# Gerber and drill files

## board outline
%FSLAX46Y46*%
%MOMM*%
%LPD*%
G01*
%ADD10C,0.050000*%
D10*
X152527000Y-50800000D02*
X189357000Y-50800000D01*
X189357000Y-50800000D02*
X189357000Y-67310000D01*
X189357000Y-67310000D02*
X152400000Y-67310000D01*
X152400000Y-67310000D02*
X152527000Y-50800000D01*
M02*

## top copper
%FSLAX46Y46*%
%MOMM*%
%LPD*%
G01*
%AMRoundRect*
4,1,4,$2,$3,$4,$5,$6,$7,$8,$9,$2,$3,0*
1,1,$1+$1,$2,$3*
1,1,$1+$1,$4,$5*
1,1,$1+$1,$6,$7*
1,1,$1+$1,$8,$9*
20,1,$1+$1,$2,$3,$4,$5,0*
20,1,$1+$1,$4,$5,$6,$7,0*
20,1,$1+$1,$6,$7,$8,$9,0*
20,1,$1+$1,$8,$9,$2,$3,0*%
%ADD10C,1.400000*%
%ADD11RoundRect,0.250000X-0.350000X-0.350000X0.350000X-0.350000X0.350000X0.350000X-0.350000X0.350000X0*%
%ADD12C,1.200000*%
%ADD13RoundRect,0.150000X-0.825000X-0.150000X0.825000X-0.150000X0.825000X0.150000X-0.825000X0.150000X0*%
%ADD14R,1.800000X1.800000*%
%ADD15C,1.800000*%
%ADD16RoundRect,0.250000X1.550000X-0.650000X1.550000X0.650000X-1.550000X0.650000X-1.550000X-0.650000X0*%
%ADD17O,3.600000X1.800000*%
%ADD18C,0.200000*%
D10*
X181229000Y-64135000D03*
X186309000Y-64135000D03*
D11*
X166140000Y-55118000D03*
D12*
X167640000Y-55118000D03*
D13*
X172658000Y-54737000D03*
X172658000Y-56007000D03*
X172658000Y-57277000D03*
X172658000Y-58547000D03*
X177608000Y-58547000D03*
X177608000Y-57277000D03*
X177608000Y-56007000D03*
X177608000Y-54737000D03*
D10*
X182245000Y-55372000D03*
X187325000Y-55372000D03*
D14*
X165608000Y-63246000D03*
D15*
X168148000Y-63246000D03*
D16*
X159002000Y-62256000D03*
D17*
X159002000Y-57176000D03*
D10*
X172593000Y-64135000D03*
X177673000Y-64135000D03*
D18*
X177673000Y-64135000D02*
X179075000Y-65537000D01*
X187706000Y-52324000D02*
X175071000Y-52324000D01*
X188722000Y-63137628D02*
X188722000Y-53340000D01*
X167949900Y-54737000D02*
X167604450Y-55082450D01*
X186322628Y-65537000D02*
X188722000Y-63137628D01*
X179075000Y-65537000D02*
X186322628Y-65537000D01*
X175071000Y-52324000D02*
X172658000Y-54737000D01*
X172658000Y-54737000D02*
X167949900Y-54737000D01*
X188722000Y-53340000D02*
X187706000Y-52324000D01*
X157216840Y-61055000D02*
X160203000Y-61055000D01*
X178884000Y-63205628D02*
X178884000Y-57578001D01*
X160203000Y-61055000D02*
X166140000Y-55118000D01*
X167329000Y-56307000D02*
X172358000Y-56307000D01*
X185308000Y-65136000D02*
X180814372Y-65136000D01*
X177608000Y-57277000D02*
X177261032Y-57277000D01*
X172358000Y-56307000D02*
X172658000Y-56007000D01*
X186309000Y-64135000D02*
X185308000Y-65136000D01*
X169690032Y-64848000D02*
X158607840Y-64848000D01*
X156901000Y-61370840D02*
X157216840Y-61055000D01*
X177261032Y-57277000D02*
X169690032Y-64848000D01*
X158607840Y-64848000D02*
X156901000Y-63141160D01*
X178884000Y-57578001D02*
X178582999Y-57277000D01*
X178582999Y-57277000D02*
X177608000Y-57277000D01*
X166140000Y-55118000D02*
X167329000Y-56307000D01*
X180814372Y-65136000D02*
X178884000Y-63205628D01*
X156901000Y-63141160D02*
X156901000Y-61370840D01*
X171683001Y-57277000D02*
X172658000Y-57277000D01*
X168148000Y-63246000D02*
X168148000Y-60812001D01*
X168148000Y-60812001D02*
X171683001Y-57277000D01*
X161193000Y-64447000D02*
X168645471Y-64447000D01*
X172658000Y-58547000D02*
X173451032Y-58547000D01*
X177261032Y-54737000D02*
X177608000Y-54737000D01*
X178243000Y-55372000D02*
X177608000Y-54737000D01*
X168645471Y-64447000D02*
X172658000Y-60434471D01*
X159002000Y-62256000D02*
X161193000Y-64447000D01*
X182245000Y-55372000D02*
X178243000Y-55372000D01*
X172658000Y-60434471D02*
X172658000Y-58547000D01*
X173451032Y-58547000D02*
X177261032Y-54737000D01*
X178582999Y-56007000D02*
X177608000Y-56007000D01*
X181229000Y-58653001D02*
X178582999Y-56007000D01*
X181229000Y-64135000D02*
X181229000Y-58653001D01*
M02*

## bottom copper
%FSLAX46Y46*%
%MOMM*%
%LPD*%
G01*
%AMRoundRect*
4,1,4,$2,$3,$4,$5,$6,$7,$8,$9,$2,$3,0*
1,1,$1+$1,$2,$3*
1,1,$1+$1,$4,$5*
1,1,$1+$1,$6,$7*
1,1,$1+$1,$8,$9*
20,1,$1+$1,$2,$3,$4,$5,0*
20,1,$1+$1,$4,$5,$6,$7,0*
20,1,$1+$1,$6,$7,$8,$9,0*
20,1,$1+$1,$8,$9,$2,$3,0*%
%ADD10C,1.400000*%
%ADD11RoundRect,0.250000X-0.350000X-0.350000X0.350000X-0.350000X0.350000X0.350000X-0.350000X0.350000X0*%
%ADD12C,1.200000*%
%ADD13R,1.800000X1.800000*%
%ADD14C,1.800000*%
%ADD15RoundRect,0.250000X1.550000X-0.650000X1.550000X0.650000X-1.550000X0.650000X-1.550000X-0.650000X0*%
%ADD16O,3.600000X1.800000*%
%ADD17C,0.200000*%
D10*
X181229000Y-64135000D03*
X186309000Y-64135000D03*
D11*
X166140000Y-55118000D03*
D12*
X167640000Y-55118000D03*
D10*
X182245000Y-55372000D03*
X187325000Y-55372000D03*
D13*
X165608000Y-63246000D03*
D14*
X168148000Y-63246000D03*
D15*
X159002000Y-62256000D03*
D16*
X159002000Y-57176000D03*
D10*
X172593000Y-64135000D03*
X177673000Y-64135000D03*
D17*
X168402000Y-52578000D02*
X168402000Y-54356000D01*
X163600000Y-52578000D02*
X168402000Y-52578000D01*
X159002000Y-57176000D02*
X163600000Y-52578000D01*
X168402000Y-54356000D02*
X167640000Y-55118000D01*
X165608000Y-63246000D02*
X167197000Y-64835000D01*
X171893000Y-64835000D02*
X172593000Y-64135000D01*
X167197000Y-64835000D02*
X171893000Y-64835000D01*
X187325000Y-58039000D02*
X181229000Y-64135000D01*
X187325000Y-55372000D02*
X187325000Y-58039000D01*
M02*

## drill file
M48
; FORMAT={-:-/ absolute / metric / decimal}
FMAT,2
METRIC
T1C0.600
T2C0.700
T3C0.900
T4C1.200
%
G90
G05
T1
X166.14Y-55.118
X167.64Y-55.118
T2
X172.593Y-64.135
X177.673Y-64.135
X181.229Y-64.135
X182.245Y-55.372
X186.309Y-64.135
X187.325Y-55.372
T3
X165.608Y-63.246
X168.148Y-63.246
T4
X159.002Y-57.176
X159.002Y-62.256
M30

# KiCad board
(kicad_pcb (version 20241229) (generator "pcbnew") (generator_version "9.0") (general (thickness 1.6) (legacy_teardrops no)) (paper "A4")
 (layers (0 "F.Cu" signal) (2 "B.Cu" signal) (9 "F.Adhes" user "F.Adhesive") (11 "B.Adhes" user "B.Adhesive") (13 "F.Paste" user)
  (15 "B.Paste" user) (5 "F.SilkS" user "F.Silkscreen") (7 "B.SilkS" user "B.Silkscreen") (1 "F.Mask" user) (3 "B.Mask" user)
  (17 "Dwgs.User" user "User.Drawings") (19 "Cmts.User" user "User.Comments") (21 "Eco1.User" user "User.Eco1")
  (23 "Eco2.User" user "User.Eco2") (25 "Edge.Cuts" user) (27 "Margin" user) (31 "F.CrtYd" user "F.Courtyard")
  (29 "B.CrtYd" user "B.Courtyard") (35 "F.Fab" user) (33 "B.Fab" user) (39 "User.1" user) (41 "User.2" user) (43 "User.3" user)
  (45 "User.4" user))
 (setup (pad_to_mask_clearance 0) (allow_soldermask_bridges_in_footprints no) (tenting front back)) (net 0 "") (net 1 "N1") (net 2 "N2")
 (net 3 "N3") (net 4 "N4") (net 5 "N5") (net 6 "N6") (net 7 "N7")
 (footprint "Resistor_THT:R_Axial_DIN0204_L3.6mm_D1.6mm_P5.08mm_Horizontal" (layer "F.Cu") (at 181.229 64.135)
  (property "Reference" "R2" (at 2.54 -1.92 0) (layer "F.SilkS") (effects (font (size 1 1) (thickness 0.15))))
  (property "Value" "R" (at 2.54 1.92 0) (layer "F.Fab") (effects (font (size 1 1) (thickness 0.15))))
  (pad "1" thru_hole circle (at 0 0) (size 1.4 1.4) (drill 0.7) (layers "*.Cu" "*.Mask") (remove_unused_layers no) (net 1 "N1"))
  (pad "2" thru_hole circle (at 5.08 0) (size 1.4 1.4) (drill 0.7) (layers "*.Cu" "*.Mask") (remove_unused_layers no) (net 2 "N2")))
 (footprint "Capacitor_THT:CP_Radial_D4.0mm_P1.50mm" (layer "F.Cu") (at 166.14 55.118)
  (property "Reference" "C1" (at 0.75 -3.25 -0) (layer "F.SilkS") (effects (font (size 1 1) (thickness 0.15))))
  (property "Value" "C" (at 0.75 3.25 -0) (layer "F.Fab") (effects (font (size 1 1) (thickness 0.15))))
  (pad "1" thru_hole roundrect (at 0 0) (size 1.2 1.2) (drill 0.6) (layers "*.Cu" "*.Mask") (remove_unused_layers no)
   (roundrect_rratio 0.208333) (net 2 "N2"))
  (pad "2" thru_hole circle (at 1.5 0) (size 1.2 1.2) (drill 0.6) (layers "*.Cu" "*.Mask") (remove_unused_layers no) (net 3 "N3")))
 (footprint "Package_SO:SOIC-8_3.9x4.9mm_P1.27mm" (layer "F.Cu") (at 175.133 56.642)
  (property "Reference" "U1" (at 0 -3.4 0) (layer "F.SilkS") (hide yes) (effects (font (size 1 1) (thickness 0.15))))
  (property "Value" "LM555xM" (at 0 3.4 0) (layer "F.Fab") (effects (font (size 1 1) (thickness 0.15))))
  (pad "1" smd roundrect (at -2.475 -1.905) (size 1.95 0.6) (layers "F.Cu" "F.Mask" "F.Paste") (roundrect_rratio 0.25) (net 3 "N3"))
  (pad "2" smd roundrect (at -2.475 -0.635) (size 1.95 0.6) (layers "F.Cu" "F.Mask" "F.Paste") (roundrect_rratio 0.25) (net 2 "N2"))
  (pad "3" smd roundrect (at -2.475 0.635) (size 1.95 0.6) (layers "F.Cu" "F.Mask" "F.Paste") (roundrect_rratio 0.25) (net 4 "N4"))
  (pad "4" smd roundrect (at -2.475 1.905) (size 1.95 0.6) (layers "F.Cu" "F.Mask" "F.Paste") (roundrect_rratio 0.25) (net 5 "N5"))
  (pad "5" smd roundrect (at 2.475 1.905) (size 1.95 0.6) (layers "F.Cu" "F.Mask" "F.Paste") (roundrect_rratio 0.25) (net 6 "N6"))
  (pad "6" smd roundrect (at 2.475 0.635) (size 1.95 0.6) (layers "F.Cu" "F.Mask" "F.Paste") (roundrect_rratio 0.25) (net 2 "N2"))
  (pad "7" smd roundrect (at 2.475 -0.635) (size 1.95 0.6) (layers "F.Cu" "F.Mask" "F.Paste") (roundrect_rratio 0.25) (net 1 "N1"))
  (pad "8" smd roundrect (at 2.475 -1.905) (size 1.95 0.6) (layers "F.Cu" "F.Mask" "F.Paste") (roundrect_rratio 0.25) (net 5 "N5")))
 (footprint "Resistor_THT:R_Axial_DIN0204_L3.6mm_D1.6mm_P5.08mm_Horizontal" (layer "F.Cu") (at 182.245 55.372)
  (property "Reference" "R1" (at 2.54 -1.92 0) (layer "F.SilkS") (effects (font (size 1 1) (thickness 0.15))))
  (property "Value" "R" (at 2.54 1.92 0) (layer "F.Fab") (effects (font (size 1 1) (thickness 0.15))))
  (pad "1" thru_hole circle (at 0 0) (size 1.4 1.4) (drill 0.7) (layers "*.Cu" "*.Mask") (remove_unused_layers no) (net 5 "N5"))
  (pad "2" thru_hole circle (at 5.08 0) (size 1.4 1.4) (drill 0.7) (layers "*.Cu" "*.Mask") (remove_unused_layers no) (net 1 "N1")))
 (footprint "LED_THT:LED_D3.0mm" (layer "F.Cu") (at 165.608 63.246)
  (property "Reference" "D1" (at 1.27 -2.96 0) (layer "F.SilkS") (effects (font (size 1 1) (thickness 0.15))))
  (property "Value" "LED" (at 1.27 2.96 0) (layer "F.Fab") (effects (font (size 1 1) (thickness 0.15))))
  (pad "1" thru_hole rect (at 0 0) (size 1.8 1.8) (drill 0.9) (layers "*.Cu" "*.Mask") (remove_unused_layers no) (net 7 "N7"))
  (pad "2" thru_hole circle (at 2.54 0) (size 1.8 1.8) (drill 0.9) (layers "*.Cu" "*.Mask") (remove_unused_layers no) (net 4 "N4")))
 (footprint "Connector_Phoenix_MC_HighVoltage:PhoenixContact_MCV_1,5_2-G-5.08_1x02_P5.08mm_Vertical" (layer "F.Cu") (at 159.002 62.256 90)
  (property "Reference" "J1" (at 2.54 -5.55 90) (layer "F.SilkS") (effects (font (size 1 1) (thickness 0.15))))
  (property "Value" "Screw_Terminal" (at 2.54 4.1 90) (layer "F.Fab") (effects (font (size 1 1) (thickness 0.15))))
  (pad "1" thru_hole roundrect (at 0 0 90) (size 1.8 3.6) (drill 1.2) (layers "*.Cu" "*.Mask") (remove_unused_layers no)
   (roundrect_rratio 0.138889) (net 5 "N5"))
  (pad "2" thru_hole oval (at 5.08 0 90) (size 1.8 3.6) (drill 1.2) (layers "*.Cu" "*.Mask") (remove_unused_layers no) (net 3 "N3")))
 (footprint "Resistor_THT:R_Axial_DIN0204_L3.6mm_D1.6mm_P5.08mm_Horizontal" (layer "F.Cu") (at 172.593 64.135)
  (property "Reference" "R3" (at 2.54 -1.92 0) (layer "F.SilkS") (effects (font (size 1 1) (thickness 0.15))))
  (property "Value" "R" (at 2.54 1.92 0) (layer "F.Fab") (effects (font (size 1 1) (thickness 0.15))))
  (pad "1" thru_hole circle (at 0 0) (size 1.4 1.4) (drill 0.7) (layers "*.Cu" "*.Mask") (remove_unused_layers no) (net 7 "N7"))
  (pad "2" thru_hole circle (at 5.08 0) (size 1.4 1.4) (drill 0.7) (layers "*.Cu" "*.Mask") (remove_unused_layers no) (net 3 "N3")))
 (gr_line (start 152.527 50.8) (end 189.357 50.8) (stroke (width 0.05) (type default)) (layer "Edge.Cuts"))
 (gr_line (start 189.357 50.8) (end 189.357 67.31) (stroke (width 0.05) (type default)) (layer "Edge.Cuts"))
 (gr_line (start 189.357 67.31) (end 152.4 67.31) (stroke (width 0.05) (type default)) (layer "Edge.Cuts"))
 (gr_line (start 152.4 67.31) (end 152.527 50.8) (stroke (width 0.05) (type default)) (layer "Edge.Cuts"))
 (segment (start 177.673 64.135) (end 179.075 65.537) (width 0.2) (layer "F.Cu") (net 3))
 (segment (start 187.706 52.324) (end 175.071 52.324) (width 0.2) (layer "F.Cu") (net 3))
 (segment (start 188.722 63.137628) (end 188.722 53.34) (width 0.2) (layer "F.Cu") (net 3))
 (segment (start 167.9499 54.737) (end 167.60445 55.08245) (width 0.2) (layer "F.Cu") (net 3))
 (segment (start 186.322628 65.537) (end 188.722 63.137628) (width 0.2) (layer "F.Cu") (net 3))
 (segment (start 179.075 65.537) (end 186.322628 65.537) (width 0.2) (layer "F.Cu") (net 3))
 (segment (start 175.071 52.324) (end 172.658 54.737) (width 0.2) (layer "F.Cu") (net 3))
 (segment (start 172.658 54.737) (end 167.9499 54.737) (width 0.2) (layer "F.Cu") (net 3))
 (segment (start 188.722 53.34) (end 187.706 52.324) (width 0.2) (layer "F.Cu") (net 3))
 (segment (start 168.402 52.578) (end 168.402 54.356) (width 0.2) (layer "B.Cu") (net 3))
 (segment (start 163.6 52.578) (end 168.402 52.578) (width 0.2) (layer "B.Cu") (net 3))
 (segment (start 159.002 57.176) (end 163.6 52.578) (width 0.2) (layer "B.Cu") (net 3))
 (segment (start 168.402 54.356) (end 167.64 55.118) (width 0.2) (layer "B.Cu") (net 3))
 (segment (start 157.21684 61.055) (end 160.203 61.055) (width 0.2) (layer "F.Cu") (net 2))
 (segment (start 178.884 63.205628) (end 178.884 57.578001) (width 0.2) (layer "F.Cu") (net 2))
 (segment (start 160.203 61.055) (end 166.14 55.118) (width 0.2) (layer "F.Cu") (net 2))
 (segment (start 167.329 56.307) (end 172.358 56.307) (width 0.2) (layer "F.Cu") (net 2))
 (segment (start 185.308 65.136) (end 180.814372 65.136) (width 0.2) (layer "F.Cu") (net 2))
 (segment (start 177.608 57.277) (end 177.261032 57.277) (width 0.2) (layer "F.Cu") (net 2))
 (segment (start 172.358 56.307) (end 172.658 56.007) (width 0.2) (layer "F.Cu") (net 2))
 (segment (start 186.309 64.135) (end 185.308 65.136) (width 0.2) (layer "F.Cu") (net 2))
 (segment (start 169.690032 64.848) (end 158.60784 64.848) (width 0.2) (layer "F.Cu") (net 2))
 (segment (start 156.901 61.37084) (end 157.21684 61.055) (width 0.2) (layer "F.Cu") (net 2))
 (segment (start 177.261032 57.277) (end 169.690032 64.848) (width 0.2) (layer "F.Cu") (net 2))
 (segment (start 158.60784 64.848) (end 156.901 63.14116) (width 0.2) (layer "F.Cu") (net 2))
 (segment (start 178.884 57.578001) (end 178.582999 57.277) (width 0.2) (layer "F.Cu") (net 2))
 (segment (start 178.582999 57.277) (end 177.608 57.277) (width 0.2) (layer "F.Cu") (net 2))
 (segment (start 166.14 55.118) (end 167.329 56.307) (width 0.2) (layer "F.Cu") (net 2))
 (segment (start 180.814372 65.136) (end 178.884 63.205628) (width 0.2) (layer "F.Cu") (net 2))
 (segment (start 156.901 63.14116) (end 156.901 61.37084) (width 0.2) (layer "F.Cu") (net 2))
 (segment (start 165.608 63.246) (end 167.197 64.835) (width 0.2) (layer "B.Cu") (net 7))
 (segment (start 171.893 64.835) (end 172.593 64.135) (width 0.2) (layer "B.Cu") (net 7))
 (segment (start 167.197 64.835) (end 171.893 64.835) (width 0.2) (layer "B.Cu") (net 7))
 (segment (start 171.683001 57.277) (end 172.658 57.277) (width 0.2) (layer "F.Cu") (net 4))
 (segment (start 168.148 63.246) (end 168.148 60.812001) (width 0.2) (layer "F.Cu") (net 4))
 (segment (start 168.148 60.812001) (end 171.683001 57.277) (width 0.2) (layer "F.Cu") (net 4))
 (segment (start 161.193 64.447) (end 168.645471 64.447) (width 0.2) (layer "F.Cu") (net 5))
 (segment (start 172.658 58.547) (end 173.451032 58.547) (width 0.2) (layer "F.Cu") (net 5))
 (segment (start 177.261032 54.737) (end 177.608 54.737) (width 0.2) (layer "F.Cu") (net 5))
 (segment (start 178.243 55.372) (end 177.608 54.737) (width 0.2) (layer "F.Cu") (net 5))
 (segment (start 168.645471 64.447) (end 172.658 60.434471) (width 0.2) (layer "F.Cu") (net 5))
 (segment (start 159.002 62.256) (end 161.193 64.447) (width 0.2) (layer "F.Cu") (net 5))
 (segment (start 182.245 55.372) (end 178.243 55.372) (width 0.2) (layer "F.Cu") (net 5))
 (segment (start 172.658 60.434471) (end 172.658 58.547) (width 0.2) (layer "F.Cu") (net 5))
 (segment (start 173.451032 58.547) (end 177.261032 54.737) (width 0.2) (layer "F.Cu") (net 5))
 (segment (start 178.582999 56.007) (end 177.608 56.007) (width 0.2) (layer "F.Cu") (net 1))
 (segment (start 181.229 58.653001) (end 178.582999 56.007) (width 0.2) (layer "F.Cu") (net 1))
 (segment (start 181.229 64.135) (end 181.229 58.653001) (width 0.2) (layer "F.Cu") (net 1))
 (segment (start 187.325 58.039) (end 181.229 64.135) (width 0.2) (layer "B.Cu") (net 1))
 (segment (start 187.325 55.372) (end 187.325 58.039) (width 0.2) (layer "B.Cu") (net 1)))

